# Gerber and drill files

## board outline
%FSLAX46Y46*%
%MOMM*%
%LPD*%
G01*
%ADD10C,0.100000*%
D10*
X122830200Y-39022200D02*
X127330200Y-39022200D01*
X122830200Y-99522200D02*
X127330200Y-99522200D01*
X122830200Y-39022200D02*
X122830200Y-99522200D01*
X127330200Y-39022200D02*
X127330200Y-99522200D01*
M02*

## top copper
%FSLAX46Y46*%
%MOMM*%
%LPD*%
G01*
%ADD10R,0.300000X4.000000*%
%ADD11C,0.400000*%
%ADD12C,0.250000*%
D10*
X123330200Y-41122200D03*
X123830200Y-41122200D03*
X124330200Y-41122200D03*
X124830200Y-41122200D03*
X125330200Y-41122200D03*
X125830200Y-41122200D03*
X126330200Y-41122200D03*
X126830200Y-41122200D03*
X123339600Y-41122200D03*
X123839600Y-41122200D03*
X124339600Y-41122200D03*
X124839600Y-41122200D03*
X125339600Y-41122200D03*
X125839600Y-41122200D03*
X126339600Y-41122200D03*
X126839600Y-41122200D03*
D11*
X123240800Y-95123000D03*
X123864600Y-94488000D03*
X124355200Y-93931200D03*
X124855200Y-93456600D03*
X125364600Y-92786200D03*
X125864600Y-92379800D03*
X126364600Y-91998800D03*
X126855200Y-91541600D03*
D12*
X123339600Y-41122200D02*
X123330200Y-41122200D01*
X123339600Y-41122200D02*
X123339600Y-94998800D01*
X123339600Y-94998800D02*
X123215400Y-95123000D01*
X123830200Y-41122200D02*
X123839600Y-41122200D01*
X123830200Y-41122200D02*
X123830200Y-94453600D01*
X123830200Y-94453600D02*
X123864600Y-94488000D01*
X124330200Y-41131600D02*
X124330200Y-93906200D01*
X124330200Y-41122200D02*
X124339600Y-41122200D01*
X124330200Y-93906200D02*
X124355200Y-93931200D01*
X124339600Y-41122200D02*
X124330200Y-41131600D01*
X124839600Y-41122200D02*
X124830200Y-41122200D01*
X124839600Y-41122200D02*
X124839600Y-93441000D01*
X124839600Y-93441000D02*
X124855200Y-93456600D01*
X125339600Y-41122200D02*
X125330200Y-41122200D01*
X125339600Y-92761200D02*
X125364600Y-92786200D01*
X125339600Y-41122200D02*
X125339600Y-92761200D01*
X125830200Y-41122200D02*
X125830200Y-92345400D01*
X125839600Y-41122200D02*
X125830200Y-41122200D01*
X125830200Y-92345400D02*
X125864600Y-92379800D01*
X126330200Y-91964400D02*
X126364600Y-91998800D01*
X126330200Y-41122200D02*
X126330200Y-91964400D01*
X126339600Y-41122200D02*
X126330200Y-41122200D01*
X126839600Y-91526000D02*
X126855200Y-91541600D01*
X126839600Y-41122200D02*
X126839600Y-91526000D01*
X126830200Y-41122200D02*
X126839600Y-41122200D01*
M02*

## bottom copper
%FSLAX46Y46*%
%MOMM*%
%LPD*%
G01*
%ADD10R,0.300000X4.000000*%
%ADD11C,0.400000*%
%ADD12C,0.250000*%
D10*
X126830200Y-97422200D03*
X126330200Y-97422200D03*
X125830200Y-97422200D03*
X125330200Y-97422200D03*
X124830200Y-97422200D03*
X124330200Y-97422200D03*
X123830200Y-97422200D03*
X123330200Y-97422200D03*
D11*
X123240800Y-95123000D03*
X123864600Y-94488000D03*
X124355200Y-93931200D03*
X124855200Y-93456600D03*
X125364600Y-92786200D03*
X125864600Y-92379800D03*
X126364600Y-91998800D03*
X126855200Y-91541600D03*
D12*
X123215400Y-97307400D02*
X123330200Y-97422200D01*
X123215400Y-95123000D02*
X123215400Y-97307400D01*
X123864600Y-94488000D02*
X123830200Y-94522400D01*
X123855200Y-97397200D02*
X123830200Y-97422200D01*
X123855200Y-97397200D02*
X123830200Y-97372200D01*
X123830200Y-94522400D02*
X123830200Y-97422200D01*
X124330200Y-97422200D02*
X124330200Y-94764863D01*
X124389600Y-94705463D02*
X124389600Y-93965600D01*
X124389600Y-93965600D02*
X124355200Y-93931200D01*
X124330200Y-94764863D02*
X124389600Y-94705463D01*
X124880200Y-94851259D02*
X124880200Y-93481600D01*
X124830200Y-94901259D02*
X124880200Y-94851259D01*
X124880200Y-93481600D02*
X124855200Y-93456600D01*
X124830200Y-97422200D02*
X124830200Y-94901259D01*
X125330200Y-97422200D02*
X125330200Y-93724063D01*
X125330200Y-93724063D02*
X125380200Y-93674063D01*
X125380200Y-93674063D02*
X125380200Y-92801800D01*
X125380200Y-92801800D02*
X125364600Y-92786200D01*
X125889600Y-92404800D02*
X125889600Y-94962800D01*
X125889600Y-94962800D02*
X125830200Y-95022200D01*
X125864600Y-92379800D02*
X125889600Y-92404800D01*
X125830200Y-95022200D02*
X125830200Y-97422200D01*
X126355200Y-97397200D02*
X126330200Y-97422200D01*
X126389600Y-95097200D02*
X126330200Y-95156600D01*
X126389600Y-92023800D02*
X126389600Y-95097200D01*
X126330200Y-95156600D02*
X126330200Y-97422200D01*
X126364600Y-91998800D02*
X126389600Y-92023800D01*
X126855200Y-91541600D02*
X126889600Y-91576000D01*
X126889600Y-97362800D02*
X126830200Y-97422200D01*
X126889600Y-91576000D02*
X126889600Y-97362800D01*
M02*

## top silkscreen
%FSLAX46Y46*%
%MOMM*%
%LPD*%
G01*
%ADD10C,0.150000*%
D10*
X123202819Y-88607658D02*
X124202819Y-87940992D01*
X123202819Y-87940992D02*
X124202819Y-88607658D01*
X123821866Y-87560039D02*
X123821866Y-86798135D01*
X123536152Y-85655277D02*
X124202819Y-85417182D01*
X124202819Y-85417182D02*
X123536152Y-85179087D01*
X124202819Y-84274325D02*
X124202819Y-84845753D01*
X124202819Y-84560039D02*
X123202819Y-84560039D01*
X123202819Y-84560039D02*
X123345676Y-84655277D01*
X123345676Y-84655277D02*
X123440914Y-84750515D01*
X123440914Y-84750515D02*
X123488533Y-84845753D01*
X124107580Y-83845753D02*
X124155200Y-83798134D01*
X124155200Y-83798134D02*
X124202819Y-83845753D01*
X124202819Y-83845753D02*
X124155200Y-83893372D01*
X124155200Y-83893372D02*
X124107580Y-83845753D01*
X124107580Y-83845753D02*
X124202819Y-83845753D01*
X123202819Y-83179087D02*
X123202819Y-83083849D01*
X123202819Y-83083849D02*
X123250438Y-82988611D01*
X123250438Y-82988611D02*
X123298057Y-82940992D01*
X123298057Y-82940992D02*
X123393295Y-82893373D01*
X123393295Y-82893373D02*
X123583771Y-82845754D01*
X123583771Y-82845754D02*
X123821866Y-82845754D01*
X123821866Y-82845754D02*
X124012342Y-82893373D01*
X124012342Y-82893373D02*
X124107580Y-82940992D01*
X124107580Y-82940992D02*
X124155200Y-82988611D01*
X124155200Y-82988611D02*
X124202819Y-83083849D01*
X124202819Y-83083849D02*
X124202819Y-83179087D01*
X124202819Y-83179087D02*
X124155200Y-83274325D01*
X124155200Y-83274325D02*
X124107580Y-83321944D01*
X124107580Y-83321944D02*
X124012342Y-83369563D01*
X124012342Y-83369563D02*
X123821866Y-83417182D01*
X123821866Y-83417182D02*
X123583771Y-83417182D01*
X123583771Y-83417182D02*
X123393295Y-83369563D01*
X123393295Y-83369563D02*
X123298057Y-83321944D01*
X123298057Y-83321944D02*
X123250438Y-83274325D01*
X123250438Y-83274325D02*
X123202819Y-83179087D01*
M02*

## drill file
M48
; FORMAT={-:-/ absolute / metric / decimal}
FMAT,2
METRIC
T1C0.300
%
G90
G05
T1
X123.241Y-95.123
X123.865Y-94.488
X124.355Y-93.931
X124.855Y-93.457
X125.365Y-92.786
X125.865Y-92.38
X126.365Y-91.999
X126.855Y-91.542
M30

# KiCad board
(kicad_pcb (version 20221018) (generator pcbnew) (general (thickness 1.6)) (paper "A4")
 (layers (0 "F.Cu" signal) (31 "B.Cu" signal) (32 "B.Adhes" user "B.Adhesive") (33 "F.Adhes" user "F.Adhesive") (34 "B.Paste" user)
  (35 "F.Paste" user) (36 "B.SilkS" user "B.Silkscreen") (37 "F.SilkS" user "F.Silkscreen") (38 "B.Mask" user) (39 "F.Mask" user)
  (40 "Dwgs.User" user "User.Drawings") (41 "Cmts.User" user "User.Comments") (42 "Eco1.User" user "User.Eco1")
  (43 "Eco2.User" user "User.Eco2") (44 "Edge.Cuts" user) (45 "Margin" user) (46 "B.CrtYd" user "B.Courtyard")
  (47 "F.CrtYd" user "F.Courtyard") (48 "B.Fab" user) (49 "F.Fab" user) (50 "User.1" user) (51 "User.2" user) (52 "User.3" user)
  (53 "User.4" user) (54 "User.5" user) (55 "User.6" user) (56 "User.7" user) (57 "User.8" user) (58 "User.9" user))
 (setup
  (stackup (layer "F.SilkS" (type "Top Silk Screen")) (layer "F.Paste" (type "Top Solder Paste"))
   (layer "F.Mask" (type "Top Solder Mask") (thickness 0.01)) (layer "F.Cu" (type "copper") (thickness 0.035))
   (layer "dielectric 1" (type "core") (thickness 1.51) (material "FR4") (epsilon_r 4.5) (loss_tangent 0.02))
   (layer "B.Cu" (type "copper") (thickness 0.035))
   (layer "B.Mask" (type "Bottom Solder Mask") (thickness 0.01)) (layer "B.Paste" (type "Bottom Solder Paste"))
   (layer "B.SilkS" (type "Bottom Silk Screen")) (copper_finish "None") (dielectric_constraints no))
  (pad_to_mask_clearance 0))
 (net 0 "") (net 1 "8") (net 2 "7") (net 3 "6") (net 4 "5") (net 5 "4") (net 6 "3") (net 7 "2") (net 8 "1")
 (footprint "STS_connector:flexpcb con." (layer "F.Cu") (at 122.8302 43.1222)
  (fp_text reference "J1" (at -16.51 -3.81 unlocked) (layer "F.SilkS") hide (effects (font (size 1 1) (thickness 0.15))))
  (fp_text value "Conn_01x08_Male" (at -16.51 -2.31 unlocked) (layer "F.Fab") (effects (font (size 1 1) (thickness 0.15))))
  (pad "1" smd rect (at 0.5 -2) (size 0.3 4) (layers "F.Cu" "F.Paste" "F.Mask") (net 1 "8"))
  (pad "2" smd rect (at 1 -2) (size 0.3 4) (layers "F.Cu" "F.Paste" "F.Mask") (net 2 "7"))
  (pad "3" smd rect (at 1.5 -2) (size 0.3 4) (layers "F.Cu" "F.Paste" "F.Mask") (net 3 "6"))
  (pad "4" smd rect (at 2 -2) (size 0.3 4) (layers "F.Cu" "F.Paste" "F.Mask") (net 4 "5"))
  (pad "5" smd rect (at 2.5 -2) (size 0.3 4) (layers "F.Cu" "F.Paste" "F.Mask") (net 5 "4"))
  (pad "6" smd rect (at 3 -2) (size 0.3 4) (layers "F.Cu" "F.Paste" "F.Mask") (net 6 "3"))
  (pad "7" smd rect (at 3.5 -2) (size 0.3 4) (layers "F.Cu" "F.Paste" "F.Mask") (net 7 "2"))
  (pad "8" smd rect (at 4 -2) (size 0.3 4) (layers "F.Cu" "F.Paste" "F.Mask") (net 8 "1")))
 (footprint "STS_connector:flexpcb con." (layer "F.Cu") (at 122.8396 43.1222) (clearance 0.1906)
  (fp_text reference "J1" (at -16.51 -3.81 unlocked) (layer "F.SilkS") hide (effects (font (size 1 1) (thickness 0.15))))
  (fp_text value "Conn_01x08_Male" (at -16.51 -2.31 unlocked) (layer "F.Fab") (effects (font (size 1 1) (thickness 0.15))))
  (pad "1" smd rect (at 0.5 -2) (size 0.3 4) (layers "F.Cu" "F.Paste" "F.Mask") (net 1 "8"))
  (pad "2" smd rect (at 1 -2) (size 0.3 4) (layers "F.Cu" "F.Paste" "F.Mask") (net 2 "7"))
  (pad "3" smd rect (at 1.5 -2) (size 0.3 4) (layers "F.Cu" "F.Paste" "F.Mask") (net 3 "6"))
  (pad "4" smd rect (at 2 -2) (size 0.3 4) (layers "F.Cu" "F.Paste" "F.Mask") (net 4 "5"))
  (pad "5" smd rect (at 2.5 -2) (size 0.3 4) (layers "F.Cu" "F.Paste" "F.Mask") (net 5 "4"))
  (pad "6" smd rect (at 3 -2) (size 0.3 4) (layers "F.Cu" "F.Paste" "F.Mask") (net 6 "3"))
  (pad "7" smd rect (at 3.5 -2) (size 0.3 4) (layers "F.Cu" "F.Paste" "F.Mask") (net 7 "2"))
  (pad "8" smd rect (at 4 -2) (size 0.3 4) (layers "F.Cu" "F.Paste" "F.Mask") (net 8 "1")))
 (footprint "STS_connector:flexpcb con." (layer "B.Cu") (at 127.3302 99.4222 180)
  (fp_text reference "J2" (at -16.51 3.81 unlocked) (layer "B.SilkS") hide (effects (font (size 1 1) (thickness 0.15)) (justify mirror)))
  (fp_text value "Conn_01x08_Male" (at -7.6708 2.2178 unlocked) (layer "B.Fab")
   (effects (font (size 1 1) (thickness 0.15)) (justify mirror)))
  (pad "1" smd rect (at 0.5 2 180) (size 0.3 4) (layers "B.Cu" "B.Paste" "B.Mask") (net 8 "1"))
  (pad "2" smd rect (at 1 2 180) (size 0.3 4) (layers "B.Cu" "B.Paste" "B.Mask") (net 7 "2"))
  (pad "3" smd rect (at 1.5 2 180) (size 0.3 4) (layers "B.Cu" "B.Paste" "B.Mask") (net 6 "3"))
  (pad "4" smd rect (at 2 2 180) (size 0.3 4) (layers "B.Cu" "B.Paste" "B.Mask") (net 5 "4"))
  (pad "5" smd rect (at 2.5 2 180) (size 0.3 4) (layers "B.Cu" "B.Paste" "B.Mask") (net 4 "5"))
  (pad "6" smd rect (at 3 2 180) (size 0.3 4) (layers "B.Cu" "B.Paste" "B.Mask") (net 3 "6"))
  (pad "7" smd rect (at 3.5 2 180) (size 0.3 4) (layers "B.Cu" "B.Paste" "B.Mask") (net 2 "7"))
  (pad "8" smd rect (at 4 2 180) (size 0.3 4) (layers "B.Cu" "B.Paste" "B.Mask") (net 1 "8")))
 (gr_line (start 122.8302 39.0222) (end 127.3302 39.0222) (stroke (width 0.1) (type solid)) (layer "Edge.Cuts"))
 (gr_line (start 122.8302 99.5222) (end 127.3302 99.5222) (stroke (width 0.1) (type solid)) (layer "Edge.Cuts"))
 (gr_line (start 122.8302 39.0222) (end 122.8302 99.5222) (stroke (width 0.1) (type solid)) (layer "Edge.Cuts"))
 (gr_line (start 127.3302 39.0222) (end 127.3302 99.5222) (stroke (width 0.1) (type solid)) (layer "Edge.Cuts"))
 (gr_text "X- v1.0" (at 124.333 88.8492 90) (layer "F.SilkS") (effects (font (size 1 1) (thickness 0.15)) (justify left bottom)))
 (segment (start 123.3396 41.1222) (end 123.3302 41.1222) (width 0.25) (layer "F.Cu") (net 1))
 (segment (start 123.3396 41.1222) (end 123.3396 94.9988) (width 0.25) (layer "F.Cu") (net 1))
 (segment (start 123.3396 94.9988) (end 123.2154 95.123) (width 0.25) (layer "F.Cu") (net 1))
 (via (at 123.2408 95.123) (size 0.4) (drill 0.3) (layers "F.Cu" "B.Cu") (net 1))
 (segment (start 123.2154 97.3074) (end 123.3302 97.4222) (width 0.25) (layer "B.Cu") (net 1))
 (segment (start 123.2154 95.123) (end 123.2154 97.3074) (width 0.25) (layer "B.Cu") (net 1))
 (segment (start 123.8302 41.1222) (end 123.8396 41.1222) (width 0.25) (layer "F.Cu") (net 2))
 (segment (start 123.8302 41.1222) (end 123.8302 94.4536) (width 0.25) (layer "F.Cu") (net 2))
 (segment (start 123.8302 94.4536) (end 123.8646 94.488) (width 0.25) (layer "F.Cu") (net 2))
 (via (at 123.8646 94.488) (size 0.4) (drill 0.3) (layers "F.Cu" "B.Cu") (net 2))
 (segment (start 123.8646 94.488) (end 123.8302 94.5224) (width 0.25) (layer "B.Cu") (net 2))
 (segment (start 123.8552 97.3972) (end 123.8302 97.4222) (width 0.25) (layer "B.Cu") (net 2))
 (segment (start 123.8552 97.3972) (end 123.8302 97.3722) (width 0.25) (layer "B.Cu") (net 2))
 (segment (start 123.8302 94.5224) (end 123.8302 97.4222) (width 0.25) (layer "B.Cu") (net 2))
 (segment (start 124.3302 41.1316) (end 124.3302 93.9062) (width 0.25) (layer "F.Cu") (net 3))
 (segment (start 124.3302 41.1222) (end 124.3396 41.1222) (width 0.25) (layer "F.Cu") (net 3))
 (segment (start 124.3302 93.9062) (end 124.3552 93.9312) (width 0.25) (layer "F.Cu") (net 3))
 (segment (start 124.3396 41.1222) (end 124.3302 41.1316) (width 0.25) (layer "F.Cu") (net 3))
 (via (at 124.3552 93.9312) (size 0.4) (drill 0.3) (layers "F.Cu" "B.Cu") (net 3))
 (segment (start 124.3302 97.4222) (end 124.3302 94.764863) (width 0.25) (layer "B.Cu") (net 3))
 (segment (start 124.3896 94.705463) (end 124.3896 93.9656) (width 0.25) (layer "B.Cu") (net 3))
 (segment (start 124.3896 93.9656) (end 124.3552 93.9312) (width 0.25) (layer "B.Cu") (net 3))
 (segment (start 124.3302 94.764863) (end 124.3896 94.705463) (width 0.25) (layer "B.Cu") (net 3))
 (segment (start 124.8396 41.1222) (end 124.8302 41.1222) (width 0.25) (layer "F.Cu") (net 4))
 (segment (start 124.8396 41.1222) (end 124.8396 93.441) (width 0.25) (layer "F.Cu") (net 4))
 (segment (start 124.8396 93.441) (end 124.8552 93.4566) (width 0.25) (layer "F.Cu") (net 4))
 (via (at 124.8552 93.4566) (size 0.4) (drill 0.3) (layers "F.Cu" "B.Cu") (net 4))
 (segment (start 124.8802 94.851259) (end 124.8802 93.4816) (width 0.25) (layer "B.Cu") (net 4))
 (segment (start 124.8302 94.901259) (end 124.8802 94.851259) (width 0.25) (layer "B.Cu") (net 4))
 (segment (start 124.8802 93.4816) (end 124.8552 93.4566) (width 0.25) (layer "B.Cu") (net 4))
 (segment (start 124.8302 97.4222) (end 124.8302 94.901259) (width 0.25) (layer "B.Cu") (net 4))
 (segment (start 125.3396 41.1222) (end 125.3302 41.1222) (width 0.25) (layer "F.Cu") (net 5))
 (segment (start 125.3396 92.7612) (end 125.3646 92.7862) (width 0.25) (layer "F.Cu") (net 5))
 (segment (start 125.3396 41.1222) (end 125.3396 92.7612) (width 0.25) (layer "F.Cu") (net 5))
 (via (at 125.3646 92.7862) (size 0.4) (drill 0.3) (layers "F.Cu" "B.Cu") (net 5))
 (segment (start 125.3302 97.4222) (end 125.3302 93.724063) (width 0.25) (layer "B.Cu") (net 5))
 (segment (start 125.3302 93.724063) (end 125.3802 93.674063) (width 0.25) (layer "B.Cu") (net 5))
 (segment (start 125.3802 93.674063) (end 125.3802 92.8018) (width 0.25) (layer "B.Cu") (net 5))
 (segment (start 125.3802 92.8018) (end 125.3646 92.7862) (width 0.25) (layer "B.Cu") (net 5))
 (segment (start 125.8302 41.1222) (end 125.8302 92.3454) (width 0.25) (layer "F.Cu") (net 6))
 (segment (start 125.8396 41.1222) (end 125.8302 41.1222) (width 0.25) (layer "F.Cu") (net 6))
 (segment (start 125.8302 92.3454) (end 125.8646 92.3798) (width 0.25) (layer "F.Cu") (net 6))
 (via (at 125.8646 92.3798) (size 0.4) (drill 0.3) (layers "F.Cu" "B.Cu") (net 6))
 (segment (start 125.8896 92.4048) (end 125.8896 94.9628) (width 0.25) (layer "B.Cu") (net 6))
 (segment (start 125.8896 94.9628) (end 125.8302 95.0222) (width 0.25) (layer "B.Cu") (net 6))
 (segment (start 125.8646 92.3798) (end 125.8896 92.4048) (width 0.25) (layer "B.Cu") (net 6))
 (segment (start 125.8302 95.0222) (end 125.8302 97.4222) (width 0.25) (layer "B.Cu") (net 6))
 (segment (start 126.3302 91.9644) (end 126.3646 91.9988) (width 0.25) (layer "F.Cu") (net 7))
 (segment (start 126.3302 41.1222) (end 126.3302 91.9644) (width 0.25) (layer "F.Cu") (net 7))
 (segment (start 126.3396 41.1222) (end 126.3302 41.1222) (width 0.25) (layer "F.Cu") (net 7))
 (via (at 126.3646 91.9988) (size 0.4) (drill 0.3) (layers "F.Cu" "B.Cu") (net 7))
 (segment (start 126.3552 97.3972) (end 126.3302 97.4222) (width 0.25) (layer "B.Cu") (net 7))
 (segment (start 126.3896 95.0972) (end 126.3302 95.1566) (width 0.25) (layer "B.Cu") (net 7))
 (segment (start 126.3896 92.0238) (end 126.3896 95.0972) (width 0.25) (layer "B.Cu") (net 7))
 (segment (start 126.3302 95.1566) (end 126.3302 97.4222) (width 0.25) (layer "B.Cu") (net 7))
 (segment (start 126.3646 91.9988) (end 126.3896 92.0238) (width 0.25) (layer "B.Cu") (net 7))
 (segment (start 126.8396 91.526) (end 126.8552 91.5416) (width 0.25) (layer "F.Cu") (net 8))
 (segment (start 126.8396 41.1222) (end 126.8396 91.526) (width 0.25) (layer "F.Cu") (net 8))
 (segment (start 126.8302 41.1222) (end 126.8396 41.1222) (width 0.25) (layer "F.Cu") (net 8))
 (via (at 126.8552 91.5416) (size 0.4) (drill 0.3) (layers "F.Cu" "B.Cu") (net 8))
 (segment (start 126.8552 91.5416) (end 126.8896 91.576) (width 0.25) (layer "B.Cu") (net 8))
 (segment (start 126.8896 97.3628) (end 126.8302 97.4222) (width 0.25) (layer "B.Cu") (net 8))
 (segment (start 126.8896 91.576) (end 126.8896 97.3628) (width 0.25) (layer "B.Cu") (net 8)))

